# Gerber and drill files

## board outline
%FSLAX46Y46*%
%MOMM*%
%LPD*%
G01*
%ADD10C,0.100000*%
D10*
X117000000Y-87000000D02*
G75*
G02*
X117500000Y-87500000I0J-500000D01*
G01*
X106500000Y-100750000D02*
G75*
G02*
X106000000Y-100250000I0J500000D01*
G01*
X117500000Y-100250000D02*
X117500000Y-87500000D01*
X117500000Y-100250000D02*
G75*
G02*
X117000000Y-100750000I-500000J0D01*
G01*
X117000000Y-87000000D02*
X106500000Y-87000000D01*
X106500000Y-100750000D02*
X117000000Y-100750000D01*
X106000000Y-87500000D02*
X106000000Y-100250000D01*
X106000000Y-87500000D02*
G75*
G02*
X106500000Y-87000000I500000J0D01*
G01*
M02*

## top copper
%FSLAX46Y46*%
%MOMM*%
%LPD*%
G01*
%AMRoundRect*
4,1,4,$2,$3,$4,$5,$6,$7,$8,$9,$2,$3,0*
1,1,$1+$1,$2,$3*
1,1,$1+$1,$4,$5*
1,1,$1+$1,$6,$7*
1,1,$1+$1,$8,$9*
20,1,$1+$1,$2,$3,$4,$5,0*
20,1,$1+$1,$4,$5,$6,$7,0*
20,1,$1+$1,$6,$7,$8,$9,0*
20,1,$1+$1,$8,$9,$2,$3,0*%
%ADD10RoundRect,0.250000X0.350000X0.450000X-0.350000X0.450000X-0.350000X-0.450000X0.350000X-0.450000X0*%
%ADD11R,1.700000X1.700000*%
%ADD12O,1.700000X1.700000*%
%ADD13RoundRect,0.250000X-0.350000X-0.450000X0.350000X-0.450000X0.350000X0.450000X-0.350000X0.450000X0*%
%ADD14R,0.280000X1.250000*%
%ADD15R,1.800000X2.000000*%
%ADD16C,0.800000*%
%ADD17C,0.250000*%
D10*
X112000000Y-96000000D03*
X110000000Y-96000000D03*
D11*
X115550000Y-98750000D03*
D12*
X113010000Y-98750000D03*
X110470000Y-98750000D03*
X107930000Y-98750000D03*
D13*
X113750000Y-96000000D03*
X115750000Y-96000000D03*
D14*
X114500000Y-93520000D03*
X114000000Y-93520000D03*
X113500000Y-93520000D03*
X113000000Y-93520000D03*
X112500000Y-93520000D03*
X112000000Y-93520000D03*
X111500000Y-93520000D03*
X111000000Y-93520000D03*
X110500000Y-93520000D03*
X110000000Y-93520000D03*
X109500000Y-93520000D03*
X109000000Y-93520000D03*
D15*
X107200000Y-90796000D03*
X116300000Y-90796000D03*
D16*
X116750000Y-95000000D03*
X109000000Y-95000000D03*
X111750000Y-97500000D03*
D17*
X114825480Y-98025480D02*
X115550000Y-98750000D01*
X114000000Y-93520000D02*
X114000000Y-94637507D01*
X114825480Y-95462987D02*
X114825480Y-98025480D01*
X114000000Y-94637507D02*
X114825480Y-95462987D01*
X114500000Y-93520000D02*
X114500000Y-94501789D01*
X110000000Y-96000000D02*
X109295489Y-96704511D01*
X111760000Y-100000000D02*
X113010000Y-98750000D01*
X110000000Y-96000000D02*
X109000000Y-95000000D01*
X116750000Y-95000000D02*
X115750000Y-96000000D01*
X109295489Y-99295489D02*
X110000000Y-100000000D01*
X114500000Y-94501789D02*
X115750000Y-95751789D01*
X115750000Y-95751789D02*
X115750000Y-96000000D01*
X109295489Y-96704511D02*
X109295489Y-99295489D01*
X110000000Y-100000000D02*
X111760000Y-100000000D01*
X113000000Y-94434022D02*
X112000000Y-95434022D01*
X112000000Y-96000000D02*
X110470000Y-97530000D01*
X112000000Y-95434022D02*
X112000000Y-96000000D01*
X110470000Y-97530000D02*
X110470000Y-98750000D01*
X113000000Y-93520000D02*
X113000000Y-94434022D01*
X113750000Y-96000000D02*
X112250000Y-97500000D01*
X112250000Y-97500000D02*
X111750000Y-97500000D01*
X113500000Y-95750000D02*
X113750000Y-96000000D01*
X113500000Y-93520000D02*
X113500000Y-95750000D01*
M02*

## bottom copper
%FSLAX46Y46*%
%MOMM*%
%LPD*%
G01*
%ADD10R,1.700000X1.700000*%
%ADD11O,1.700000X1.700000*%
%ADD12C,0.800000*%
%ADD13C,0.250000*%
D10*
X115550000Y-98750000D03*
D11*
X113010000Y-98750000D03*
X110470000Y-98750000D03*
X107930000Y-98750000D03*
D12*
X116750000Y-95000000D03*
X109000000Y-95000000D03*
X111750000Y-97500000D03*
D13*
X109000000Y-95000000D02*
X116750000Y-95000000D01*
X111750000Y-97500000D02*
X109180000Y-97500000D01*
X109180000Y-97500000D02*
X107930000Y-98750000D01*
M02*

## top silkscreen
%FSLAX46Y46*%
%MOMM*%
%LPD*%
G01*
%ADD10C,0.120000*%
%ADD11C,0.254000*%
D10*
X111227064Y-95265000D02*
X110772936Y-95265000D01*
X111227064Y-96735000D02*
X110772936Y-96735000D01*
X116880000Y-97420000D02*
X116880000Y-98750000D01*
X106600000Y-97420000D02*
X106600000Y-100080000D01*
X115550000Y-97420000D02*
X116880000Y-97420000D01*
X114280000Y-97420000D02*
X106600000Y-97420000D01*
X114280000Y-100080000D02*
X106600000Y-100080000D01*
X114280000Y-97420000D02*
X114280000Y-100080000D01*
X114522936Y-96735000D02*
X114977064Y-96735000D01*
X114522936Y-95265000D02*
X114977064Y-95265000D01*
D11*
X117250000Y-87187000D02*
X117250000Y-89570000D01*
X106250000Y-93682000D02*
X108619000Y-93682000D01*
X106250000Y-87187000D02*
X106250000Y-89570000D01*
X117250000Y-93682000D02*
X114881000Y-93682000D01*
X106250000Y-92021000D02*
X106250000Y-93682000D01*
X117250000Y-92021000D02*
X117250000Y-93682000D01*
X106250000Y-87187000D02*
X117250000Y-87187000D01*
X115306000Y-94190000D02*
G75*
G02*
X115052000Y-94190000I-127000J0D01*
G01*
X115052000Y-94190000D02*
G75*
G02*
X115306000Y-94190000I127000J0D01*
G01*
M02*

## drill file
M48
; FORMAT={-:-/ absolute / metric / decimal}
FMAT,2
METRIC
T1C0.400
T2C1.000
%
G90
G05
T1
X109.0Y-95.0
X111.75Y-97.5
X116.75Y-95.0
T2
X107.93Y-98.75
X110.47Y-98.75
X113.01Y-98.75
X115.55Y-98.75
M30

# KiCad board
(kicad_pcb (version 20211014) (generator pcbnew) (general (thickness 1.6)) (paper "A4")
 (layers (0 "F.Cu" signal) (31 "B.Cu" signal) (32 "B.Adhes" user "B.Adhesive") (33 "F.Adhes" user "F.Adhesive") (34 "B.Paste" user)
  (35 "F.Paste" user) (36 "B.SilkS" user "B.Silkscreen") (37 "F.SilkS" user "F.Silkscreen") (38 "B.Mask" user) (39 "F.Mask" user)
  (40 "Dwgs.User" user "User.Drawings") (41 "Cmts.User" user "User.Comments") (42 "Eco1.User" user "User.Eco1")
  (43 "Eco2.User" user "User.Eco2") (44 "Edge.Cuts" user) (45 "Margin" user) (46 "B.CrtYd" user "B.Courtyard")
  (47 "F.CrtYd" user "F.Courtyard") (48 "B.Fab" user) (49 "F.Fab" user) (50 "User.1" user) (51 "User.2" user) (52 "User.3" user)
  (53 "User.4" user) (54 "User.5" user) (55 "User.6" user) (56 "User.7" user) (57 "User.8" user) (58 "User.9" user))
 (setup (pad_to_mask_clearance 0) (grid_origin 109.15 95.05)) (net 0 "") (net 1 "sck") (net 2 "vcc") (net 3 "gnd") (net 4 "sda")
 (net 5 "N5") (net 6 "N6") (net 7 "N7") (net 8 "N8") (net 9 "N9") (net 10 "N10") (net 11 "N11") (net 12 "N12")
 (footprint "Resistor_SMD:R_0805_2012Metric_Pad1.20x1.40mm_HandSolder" (layer "F.Cu") (at 111 96 180)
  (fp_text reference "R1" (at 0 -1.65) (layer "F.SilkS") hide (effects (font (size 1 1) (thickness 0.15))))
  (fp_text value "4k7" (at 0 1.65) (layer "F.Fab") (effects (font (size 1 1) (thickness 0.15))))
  (fp_line (start -0.227064 0.735) (end 0.227064 0.735) (layer "F.SilkS") (width 0.12))
  (fp_line (start -0.227064 -0.735) (end 0.227064 -0.735) (layer "F.SilkS") (width 0.12))
  (pad "1" smd roundrect (at -1 0 180) (size 1.2 1.4) (layers "F.Cu" "F.Paste" "F.Mask") (roundrect_rratio 0.2083333333) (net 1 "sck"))
  (pad "2" smd roundrect (at 1 0 180) (size 1.2 1.4) (layers "F.Cu" "F.Paste" "F.Mask") (roundrect_rratio 0.2083333333) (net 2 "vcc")))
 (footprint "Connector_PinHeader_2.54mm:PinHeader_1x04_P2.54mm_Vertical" (layer "F.Cu") (at 115.55 98.75 -90)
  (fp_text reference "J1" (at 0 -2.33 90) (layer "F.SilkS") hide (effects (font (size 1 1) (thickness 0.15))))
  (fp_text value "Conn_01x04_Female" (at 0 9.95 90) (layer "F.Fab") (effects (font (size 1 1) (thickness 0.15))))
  (fp_line (start -1.33 -1.33) (end 0 -1.33) (layer "F.SilkS") (width 0.12))
  (fp_line (start -1.33 8.95) (end 1.33 8.95) (layer "F.SilkS") (width 0.12))
  (fp_line (start -1.33 0) (end -1.33 -1.33) (layer "F.SilkS") (width 0.12))
  (fp_line (start -1.33 1.27) (end -1.33 8.95) (layer "F.SilkS") (width 0.12))
  (fp_line (start 1.33 1.27) (end 1.33 8.95) (layer "F.SilkS") (width 0.12))
  (fp_line (start -1.33 1.27) (end 1.33 1.27) (layer "F.SilkS") (width 0.12))
  (pad "1" thru_hole rect (at 0 0 270) (size 1.7 1.7) (drill 1) (layers *.Cu *.Mask) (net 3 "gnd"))
  (pad "2" thru_hole oval (at 0 2.54 270) (size 1.7 1.7) (drill 1) (layers *.Cu *.Mask) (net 2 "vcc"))
  (pad "3" thru_hole oval (at 0 5.08 270) (size 1.7 1.7) (drill 1) (layers *.Cu *.Mask) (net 1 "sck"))
  (pad "4" thru_hole oval (at 0 7.62 270) (size 1.7 1.7) (drill 1) (layers *.Cu *.Mask) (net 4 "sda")))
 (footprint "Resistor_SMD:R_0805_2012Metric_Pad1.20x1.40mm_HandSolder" (layer "F.Cu") (at 114.75 96)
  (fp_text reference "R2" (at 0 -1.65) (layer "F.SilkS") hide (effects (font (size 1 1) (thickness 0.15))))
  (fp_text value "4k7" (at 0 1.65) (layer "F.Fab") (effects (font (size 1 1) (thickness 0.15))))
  (fp_line (start -0.227064 0.735) (end 0.227064 0.735) (layer "F.SilkS") (width 0.12))
  (fp_line (start -0.227064 -0.735) (end 0.227064 -0.735) (layer "F.SilkS") (width 0.12))
  (pad "1" smd roundrect (at -1 0) (size 1.2 1.4) (layers "F.Cu" "F.Paste" "F.Mask") (roundrect_rratio 0.2083333333) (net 4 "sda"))
  (pad "2" smd roundrect (at 1 0) (size 1.2 1.4) (layers "F.Cu" "F.Paste" "F.Mask") (roundrect_rratio 0.2083333333) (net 2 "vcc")))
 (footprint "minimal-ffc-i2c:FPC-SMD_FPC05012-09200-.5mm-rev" (layer "F.Cu") (at 111.75 92.158 180)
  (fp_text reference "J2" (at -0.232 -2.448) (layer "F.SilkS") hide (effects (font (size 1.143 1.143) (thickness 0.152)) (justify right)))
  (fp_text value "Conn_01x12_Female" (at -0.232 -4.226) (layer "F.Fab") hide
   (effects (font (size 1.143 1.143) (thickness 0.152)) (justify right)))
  (fp_line (start -5.5 4.971) (end -5.5 2.588) (layer "F.SilkS") (width 0.254))
  (fp_line (start 5.5 -1.524) (end 3.131 -1.524) (layer "F.SilkS") (width 0.254))
  (fp_line (start 5.5 4.971) (end 5.5 2.588) (layer "F.SilkS") (width 0.254))
  (fp_line (start -5.5 -1.524) (end -3.131 -1.524) (layer "F.SilkS") (width 0.254))
  (fp_line (start 5.5 0.137) (end 5.5 -1.524) (layer "F.SilkS") (width 0.254))
  (fp_line (start -5.5 0.137) (end -5.5 -1.524) (layer "F.SilkS") (width 0.254))
  (fp_line (start 5.5 4.971) (end -5.5 4.971) (layer "F.SilkS") (width 0.254))
  (fp_circle (center -3.429 -2.032) (end -3.302 -2.032) (layer "F.SilkS") (width 0.254) (fill none))
  (pad "1" smd rect (at -2.75 -1.362 180) (size 0.28 1.25) (layers "F.Cu" "F.Paste" "F.Mask") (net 2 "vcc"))
  (pad "2" smd rect (at -2.25 -1.362 180) (size 0.28 1.25) (layers "F.Cu" "F.Paste" "F.Mask") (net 3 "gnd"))
  (pad "3" smd rect (at -1.75 -1.362 180) (size 0.28 1.25) (layers "F.Cu" "F.Paste" "F.Mask") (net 4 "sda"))
  (pad "4" smd rect (at -1.25 -1.362 180) (size 0.28 1.25) (layers "F.Cu" "F.Paste" "F.Mask") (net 1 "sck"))
  (pad "5" smd rect (at -0.75 -1.362 180) (size 0.28 1.25) (layers "F.Cu" "F.Paste" "F.Mask") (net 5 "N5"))
  (pad "6" smd rect (at -0.25 -1.362 180) (size 0.28 1.25) (layers "F.Cu" "F.Paste" "F.Mask") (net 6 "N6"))
  (pad "7" smd rect (at 0.25 -1.362 180) (size 0.28 1.25) (layers "F.Cu" "F.Paste" "F.Mask") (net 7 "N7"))
  (pad "8" smd rect (at 0.75 -1.362 180) (size 0.28 1.25) (layers "F.Cu" "F.Paste" "F.Mask") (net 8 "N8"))
  (pad "9" smd rect (at 1.25 -1.362 180) (size 0.28 1.25) (layers "F.Cu" "F.Paste" "F.Mask") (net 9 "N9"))
  (pad "10" smd rect (at 1.75 -1.362 180) (size 0.28 1.25) (layers "F.Cu" "F.Paste" "F.Mask") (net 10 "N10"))
  (pad "11" smd rect (at 2.25 -1.362 180) (size 0.28 1.25) (layers "F.Cu" "F.Paste" "F.Mask") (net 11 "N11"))
  (pad "12" smd rect (at 2.75 -1.362 180) (size 0.28 1.25) (layers "F.Cu" "F.Paste" "F.Mask") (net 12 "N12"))
  (pad "13" smd rect (at 4.55 1.362 180) (size 1.8 2) (layers "F.Cu" "F.Paste" "F.Mask"))
  (pad "14" smd rect (at -4.55 1.362 180) (size 1.8 2) (layers "F.Cu" "F.Paste" "F.Mask")))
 (gr_arc (start 117 87) (mid 117.353553 87.146447) (end 117.5 87.5) (layer "Edge.Cuts") (width 0.1))
 (gr_arc (start 106.5 100.75) (mid 106.146447 100.603553) (end 106 100.25) (layer "Edge.Cuts") (width 0.1))
 (gr_line (start 117.5 100.25) (end 117.5 87.5) (layer "Edge.Cuts") (width 0.1))
 (gr_arc (start 117.5 100.25) (mid 117.353553 100.603553) (end 117 100.75) (layer "Edge.Cuts") (width 0.1))
 (gr_line (start 117 87) (end 106.5 87) (layer "Edge.Cuts") (width 0.1))
 (gr_line (start 106.5 100.75) (end 117 100.75) (layer "Edge.Cuts") (width 0.1))
 (gr_line (start 106 87.5) (end 106 100.25) (layer "Edge.Cuts") (width 0.1))
 (gr_arc (start 106 87.5) (mid 106.146447 87.146447) (end 106.5 87) (layer "Edge.Cuts") (width 0.1))
 (segment (start 114.82548 98.02548) (end 115.55 98.75) (width 0.25) (layer "F.Cu") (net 3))
 (segment (start 114 93.52) (end 114 94.637507) (width 0.25) (layer "F.Cu") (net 3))
 (segment (start 114.82548 95.462987) (end 114.82548 98.02548) (width 0.25) (layer "F.Cu") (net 3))
 (segment (start 114 94.637507) (end 114.82548 95.462987) (width 0.25) (layer "F.Cu") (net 3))
 (segment (start 114.5 93.52) (end 114.5 94.501789) (width 0.25) (layer "F.Cu") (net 2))
 (segment (start 110 96) (end 109.295489 96.704511) (width 0.25) (layer "F.Cu") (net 2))
 (segment (start 111.76 100) (end 113.01 98.75) (width 0.25) (layer "F.Cu") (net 2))
 (segment (start 110 96) (end 109 95) (width 0.25) (layer "F.Cu") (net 2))
 (segment (start 116.75 95) (end 115.75 96) (width 0.25) (layer "F.Cu") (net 2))
 (segment (start 109.295489 99.295489) (end 110 100) (width 0.25) (layer "F.Cu") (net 2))
 (segment (start 114.5 94.501789) (end 115.75 95.751789) (width 0.25) (layer "F.Cu") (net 2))
 (segment (start 115.75 95.751789) (end 115.75 96) (width 0.25) (layer "F.Cu") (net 2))
 (segment (start 109.295489 96.704511) (end 109.295489 99.295489) (width 0.25) (layer "F.Cu") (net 2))
 (segment (start 110 100) (end 111.76 100) (width 0.25) (layer "F.Cu") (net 2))
 (via (at 116.75 95) (size 0.8) (drill 0.4) (layers "F.Cu" "B.Cu") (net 2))
 (via (at 109 95) (size 0.8) (drill 0.4) (layers "F.Cu" "B.Cu") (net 2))
 (segment (start 109 95) (end 116.75 95) (width 0.25) (layer "B.Cu") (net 2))
 (segment (start 113 94.434022) (end 112 95.434022) (width 0.25) (layer "F.Cu") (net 1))
 (segment (start 112 96) (end 110.47 97.53) (width 0.25) (layer "F.Cu") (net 1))
 (segment (start 112 95.434022) (end 112 96) (width 0.25) (layer "F.Cu") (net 1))
 (segment (start 110.47 97.53) (end 110.47 98.75) (width 0.25) (layer "F.Cu") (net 1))
 (segment (start 113 93.52) (end 113 94.434022) (width 0.25) (layer "F.Cu") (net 1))
 (segment (start 113.75 96) (end 112.25 97.5) (width 0.25) (layer "F.Cu") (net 4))
 (segment (start 112.25 97.5) (end 111.75 97.5) (width 0.25) (layer "F.Cu") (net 4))
 (segment (start 113.5 95.75) (end 113.75 96) (width 0.25) (layer "F.Cu") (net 4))
 (segment (start 113.5 93.52) (end 113.5 95.75) (width 0.25) (layer "F.Cu") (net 4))
 (via (at 111.75 97.5) (size 0.8) (drill 0.4) (layers "F.Cu" "B.Cu") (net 4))
 (segment (start 111.75 97.5) (end 109.18 97.5) (width 0.25) (layer "B.Cu") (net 4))
 (segment (start 109.18 97.5) (end 107.93 98.75) (width 0.25) (layer "B.Cu") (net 4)))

